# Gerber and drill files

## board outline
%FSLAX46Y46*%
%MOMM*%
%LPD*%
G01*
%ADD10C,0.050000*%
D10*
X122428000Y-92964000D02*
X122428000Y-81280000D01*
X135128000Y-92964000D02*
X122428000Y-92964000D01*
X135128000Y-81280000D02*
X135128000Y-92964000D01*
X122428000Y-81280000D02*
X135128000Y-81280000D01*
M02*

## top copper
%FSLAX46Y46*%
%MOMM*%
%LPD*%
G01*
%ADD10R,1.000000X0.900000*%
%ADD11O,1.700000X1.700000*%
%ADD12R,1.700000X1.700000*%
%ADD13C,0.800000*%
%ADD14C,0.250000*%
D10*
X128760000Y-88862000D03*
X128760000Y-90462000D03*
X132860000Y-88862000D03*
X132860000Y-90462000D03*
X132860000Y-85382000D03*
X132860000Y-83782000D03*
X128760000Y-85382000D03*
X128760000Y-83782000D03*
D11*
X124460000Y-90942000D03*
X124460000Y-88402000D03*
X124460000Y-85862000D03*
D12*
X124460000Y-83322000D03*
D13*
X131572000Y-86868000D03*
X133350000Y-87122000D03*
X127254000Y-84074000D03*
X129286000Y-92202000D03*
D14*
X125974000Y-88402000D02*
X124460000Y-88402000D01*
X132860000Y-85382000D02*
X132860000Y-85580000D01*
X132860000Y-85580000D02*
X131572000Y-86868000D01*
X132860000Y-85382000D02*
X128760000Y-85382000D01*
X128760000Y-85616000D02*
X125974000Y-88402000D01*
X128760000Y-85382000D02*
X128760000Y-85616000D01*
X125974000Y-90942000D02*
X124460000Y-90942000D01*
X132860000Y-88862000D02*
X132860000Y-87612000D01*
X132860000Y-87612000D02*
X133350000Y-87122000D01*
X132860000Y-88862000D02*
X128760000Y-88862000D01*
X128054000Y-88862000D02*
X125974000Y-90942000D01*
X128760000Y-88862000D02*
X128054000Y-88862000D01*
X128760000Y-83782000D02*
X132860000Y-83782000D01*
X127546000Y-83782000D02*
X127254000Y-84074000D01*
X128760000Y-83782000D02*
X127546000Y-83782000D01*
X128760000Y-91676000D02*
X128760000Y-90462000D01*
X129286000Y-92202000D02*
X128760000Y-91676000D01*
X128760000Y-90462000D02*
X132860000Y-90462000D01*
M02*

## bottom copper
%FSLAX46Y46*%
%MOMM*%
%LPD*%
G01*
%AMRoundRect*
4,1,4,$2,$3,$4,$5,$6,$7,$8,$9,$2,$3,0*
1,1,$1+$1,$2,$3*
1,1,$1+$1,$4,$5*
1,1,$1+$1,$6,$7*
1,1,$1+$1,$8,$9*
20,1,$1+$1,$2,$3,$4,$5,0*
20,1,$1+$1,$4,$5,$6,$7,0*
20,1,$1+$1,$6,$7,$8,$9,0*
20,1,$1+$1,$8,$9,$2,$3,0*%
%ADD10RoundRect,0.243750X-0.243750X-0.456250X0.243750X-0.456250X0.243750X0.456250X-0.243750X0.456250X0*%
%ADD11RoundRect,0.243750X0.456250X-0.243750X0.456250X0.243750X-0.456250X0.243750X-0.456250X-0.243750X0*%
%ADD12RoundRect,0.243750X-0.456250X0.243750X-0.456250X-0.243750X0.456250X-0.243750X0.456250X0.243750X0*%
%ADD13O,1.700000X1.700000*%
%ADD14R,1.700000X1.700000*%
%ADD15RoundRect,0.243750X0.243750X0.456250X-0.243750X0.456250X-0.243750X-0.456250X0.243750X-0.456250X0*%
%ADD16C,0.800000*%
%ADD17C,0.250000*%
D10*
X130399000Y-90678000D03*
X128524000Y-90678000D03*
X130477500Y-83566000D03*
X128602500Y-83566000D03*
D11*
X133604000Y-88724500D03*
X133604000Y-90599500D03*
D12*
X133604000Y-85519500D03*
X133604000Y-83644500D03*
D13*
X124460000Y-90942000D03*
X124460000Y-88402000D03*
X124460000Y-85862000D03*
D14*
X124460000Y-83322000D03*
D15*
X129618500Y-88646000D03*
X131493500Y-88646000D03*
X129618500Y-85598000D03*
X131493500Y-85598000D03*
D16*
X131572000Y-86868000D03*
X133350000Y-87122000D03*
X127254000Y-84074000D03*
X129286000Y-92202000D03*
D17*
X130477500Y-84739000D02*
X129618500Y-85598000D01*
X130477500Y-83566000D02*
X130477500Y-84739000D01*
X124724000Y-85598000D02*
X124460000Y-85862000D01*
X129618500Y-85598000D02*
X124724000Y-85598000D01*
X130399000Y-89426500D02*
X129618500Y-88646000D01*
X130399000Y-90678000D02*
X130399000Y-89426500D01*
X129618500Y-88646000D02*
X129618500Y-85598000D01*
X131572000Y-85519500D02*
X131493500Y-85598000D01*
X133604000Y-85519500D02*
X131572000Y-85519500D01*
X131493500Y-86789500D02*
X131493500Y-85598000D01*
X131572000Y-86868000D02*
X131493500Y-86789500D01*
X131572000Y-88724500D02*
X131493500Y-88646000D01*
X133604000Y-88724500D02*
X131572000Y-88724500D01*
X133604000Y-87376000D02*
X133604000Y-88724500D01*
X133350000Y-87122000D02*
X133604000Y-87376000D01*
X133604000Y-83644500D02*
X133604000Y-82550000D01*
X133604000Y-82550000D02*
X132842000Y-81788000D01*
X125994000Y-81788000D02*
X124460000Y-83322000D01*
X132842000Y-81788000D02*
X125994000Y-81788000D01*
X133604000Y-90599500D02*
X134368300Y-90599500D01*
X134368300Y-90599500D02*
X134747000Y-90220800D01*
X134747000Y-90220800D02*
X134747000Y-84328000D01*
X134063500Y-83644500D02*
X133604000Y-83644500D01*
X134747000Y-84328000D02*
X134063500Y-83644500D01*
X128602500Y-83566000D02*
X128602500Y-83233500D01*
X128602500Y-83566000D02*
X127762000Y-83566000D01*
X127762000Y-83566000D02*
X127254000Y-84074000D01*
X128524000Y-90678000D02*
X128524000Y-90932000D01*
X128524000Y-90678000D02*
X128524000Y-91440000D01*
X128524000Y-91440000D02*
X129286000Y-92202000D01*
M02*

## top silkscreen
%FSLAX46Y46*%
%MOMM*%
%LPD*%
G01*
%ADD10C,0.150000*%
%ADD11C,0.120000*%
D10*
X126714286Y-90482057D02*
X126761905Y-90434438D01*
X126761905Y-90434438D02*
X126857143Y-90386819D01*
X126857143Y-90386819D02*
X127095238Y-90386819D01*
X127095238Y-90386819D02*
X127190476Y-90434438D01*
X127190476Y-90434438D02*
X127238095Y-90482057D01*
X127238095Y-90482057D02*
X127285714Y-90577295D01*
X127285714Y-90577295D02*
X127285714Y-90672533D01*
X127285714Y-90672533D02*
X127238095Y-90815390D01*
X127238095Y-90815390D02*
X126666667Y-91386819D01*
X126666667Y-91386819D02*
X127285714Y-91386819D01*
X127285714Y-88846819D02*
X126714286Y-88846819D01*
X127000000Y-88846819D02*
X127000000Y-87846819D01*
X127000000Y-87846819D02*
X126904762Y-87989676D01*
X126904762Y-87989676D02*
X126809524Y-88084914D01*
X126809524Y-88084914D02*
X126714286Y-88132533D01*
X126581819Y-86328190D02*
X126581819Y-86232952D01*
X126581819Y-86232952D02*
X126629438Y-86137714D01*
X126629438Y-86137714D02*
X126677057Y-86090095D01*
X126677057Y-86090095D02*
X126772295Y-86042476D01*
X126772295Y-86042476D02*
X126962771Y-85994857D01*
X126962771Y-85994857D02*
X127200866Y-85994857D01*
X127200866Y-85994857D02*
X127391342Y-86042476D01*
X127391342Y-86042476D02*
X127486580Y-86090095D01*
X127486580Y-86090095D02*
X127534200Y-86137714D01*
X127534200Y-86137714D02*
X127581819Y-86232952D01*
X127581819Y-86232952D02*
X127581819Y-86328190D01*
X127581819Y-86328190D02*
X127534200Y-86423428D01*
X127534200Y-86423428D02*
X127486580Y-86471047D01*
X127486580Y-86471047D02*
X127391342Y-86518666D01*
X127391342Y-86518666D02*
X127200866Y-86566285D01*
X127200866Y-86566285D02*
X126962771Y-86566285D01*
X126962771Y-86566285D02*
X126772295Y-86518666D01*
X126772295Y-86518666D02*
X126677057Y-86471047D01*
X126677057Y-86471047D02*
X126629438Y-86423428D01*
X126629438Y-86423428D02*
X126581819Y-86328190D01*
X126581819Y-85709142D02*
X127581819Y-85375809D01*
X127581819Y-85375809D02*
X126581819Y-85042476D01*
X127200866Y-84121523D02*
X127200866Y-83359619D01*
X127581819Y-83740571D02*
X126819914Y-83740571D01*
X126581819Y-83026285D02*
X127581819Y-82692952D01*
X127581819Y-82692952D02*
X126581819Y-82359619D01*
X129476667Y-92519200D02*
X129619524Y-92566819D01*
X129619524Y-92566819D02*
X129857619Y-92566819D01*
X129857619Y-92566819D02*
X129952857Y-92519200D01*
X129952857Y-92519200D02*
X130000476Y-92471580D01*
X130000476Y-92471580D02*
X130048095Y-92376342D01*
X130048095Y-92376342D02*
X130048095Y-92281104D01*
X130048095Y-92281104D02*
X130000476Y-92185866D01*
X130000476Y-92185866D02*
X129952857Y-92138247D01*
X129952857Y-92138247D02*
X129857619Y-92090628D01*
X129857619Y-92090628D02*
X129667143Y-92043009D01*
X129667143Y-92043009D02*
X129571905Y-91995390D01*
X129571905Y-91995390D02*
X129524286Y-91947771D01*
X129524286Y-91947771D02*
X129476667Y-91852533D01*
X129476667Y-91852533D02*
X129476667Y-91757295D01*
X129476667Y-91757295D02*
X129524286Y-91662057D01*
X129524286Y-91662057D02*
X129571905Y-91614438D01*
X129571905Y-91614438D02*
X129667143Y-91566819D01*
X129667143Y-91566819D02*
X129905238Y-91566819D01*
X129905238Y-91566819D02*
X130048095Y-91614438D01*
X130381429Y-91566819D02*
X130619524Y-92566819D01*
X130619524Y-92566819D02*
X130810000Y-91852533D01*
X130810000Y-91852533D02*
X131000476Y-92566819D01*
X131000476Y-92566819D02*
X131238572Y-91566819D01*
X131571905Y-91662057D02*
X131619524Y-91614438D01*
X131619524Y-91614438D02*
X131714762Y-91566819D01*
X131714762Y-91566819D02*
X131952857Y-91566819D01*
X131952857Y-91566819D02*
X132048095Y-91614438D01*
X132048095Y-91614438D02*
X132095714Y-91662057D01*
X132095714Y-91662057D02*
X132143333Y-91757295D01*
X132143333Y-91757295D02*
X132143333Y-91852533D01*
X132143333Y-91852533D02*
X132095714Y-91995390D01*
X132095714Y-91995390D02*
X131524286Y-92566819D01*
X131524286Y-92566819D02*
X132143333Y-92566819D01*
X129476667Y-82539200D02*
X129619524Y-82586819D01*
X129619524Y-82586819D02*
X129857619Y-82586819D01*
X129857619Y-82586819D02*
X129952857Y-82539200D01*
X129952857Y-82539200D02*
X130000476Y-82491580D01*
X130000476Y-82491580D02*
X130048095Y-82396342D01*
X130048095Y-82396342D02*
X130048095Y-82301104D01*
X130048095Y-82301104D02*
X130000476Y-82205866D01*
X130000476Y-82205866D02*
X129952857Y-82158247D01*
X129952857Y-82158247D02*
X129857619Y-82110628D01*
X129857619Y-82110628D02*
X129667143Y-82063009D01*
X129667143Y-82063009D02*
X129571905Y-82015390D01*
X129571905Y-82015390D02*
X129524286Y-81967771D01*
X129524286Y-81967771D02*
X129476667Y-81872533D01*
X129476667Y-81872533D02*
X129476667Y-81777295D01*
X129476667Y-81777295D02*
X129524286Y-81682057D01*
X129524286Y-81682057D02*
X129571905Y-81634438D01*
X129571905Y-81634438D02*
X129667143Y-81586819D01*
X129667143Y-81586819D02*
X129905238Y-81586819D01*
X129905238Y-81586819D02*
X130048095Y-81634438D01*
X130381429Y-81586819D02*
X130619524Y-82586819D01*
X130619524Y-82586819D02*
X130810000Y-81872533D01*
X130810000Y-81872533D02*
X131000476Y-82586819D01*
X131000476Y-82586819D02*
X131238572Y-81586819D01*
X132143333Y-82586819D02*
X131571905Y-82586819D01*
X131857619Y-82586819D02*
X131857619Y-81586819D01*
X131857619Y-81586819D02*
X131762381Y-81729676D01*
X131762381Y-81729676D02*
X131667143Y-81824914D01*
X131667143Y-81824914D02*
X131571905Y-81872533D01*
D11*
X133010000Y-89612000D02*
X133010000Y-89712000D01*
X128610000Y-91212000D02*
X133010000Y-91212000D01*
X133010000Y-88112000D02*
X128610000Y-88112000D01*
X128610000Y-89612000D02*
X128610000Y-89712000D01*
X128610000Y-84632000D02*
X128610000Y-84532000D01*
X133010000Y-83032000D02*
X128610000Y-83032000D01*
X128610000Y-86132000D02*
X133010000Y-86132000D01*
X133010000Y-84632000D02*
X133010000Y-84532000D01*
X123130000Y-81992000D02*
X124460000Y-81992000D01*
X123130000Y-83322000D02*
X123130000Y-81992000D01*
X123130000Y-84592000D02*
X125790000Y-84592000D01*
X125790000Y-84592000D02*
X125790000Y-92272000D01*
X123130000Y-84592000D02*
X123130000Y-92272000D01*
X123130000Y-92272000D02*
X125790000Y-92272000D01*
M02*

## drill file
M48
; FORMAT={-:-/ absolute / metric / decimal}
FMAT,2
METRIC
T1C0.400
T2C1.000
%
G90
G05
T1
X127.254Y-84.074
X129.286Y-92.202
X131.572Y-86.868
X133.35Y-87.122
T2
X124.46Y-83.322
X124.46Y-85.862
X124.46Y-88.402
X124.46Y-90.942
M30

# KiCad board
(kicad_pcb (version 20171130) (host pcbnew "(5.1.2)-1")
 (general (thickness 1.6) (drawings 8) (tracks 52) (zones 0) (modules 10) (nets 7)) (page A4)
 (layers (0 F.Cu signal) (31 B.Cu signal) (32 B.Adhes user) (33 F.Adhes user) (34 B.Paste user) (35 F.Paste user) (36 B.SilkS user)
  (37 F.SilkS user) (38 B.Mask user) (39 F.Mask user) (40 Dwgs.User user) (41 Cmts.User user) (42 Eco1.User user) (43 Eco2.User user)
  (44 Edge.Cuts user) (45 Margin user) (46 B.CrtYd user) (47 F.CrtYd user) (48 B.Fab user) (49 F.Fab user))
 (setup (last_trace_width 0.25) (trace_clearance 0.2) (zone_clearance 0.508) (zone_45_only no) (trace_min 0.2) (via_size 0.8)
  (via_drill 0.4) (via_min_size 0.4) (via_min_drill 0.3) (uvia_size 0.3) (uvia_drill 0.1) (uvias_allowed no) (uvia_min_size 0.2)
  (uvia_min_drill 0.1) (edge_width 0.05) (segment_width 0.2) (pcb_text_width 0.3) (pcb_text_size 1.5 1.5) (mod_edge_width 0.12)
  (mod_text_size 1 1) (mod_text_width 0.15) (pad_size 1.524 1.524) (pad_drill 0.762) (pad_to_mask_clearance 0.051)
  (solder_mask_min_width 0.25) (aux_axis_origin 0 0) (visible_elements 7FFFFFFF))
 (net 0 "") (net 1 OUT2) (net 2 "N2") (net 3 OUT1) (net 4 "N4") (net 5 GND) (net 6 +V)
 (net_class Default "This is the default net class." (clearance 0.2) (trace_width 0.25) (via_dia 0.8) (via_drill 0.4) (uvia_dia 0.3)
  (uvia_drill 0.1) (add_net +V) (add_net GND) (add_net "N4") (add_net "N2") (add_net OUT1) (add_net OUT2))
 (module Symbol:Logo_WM (layer B.Cu) (at 127.381 87.122 270)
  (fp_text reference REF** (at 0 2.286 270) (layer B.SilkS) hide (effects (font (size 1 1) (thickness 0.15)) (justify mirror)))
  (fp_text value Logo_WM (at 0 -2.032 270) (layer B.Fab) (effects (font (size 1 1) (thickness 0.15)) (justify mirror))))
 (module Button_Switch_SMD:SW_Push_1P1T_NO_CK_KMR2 (layer F.Cu) (at 130.81 89.662 180)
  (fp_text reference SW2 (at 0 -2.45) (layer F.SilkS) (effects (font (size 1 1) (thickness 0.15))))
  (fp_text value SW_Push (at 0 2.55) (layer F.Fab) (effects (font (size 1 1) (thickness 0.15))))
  (fp_line (start -2.2 0.05) (end -2.2 -0.05) (layer F.SilkS) (width 0.12))
  (fp_line (start 2.2 -1.55) (end -2.2 -1.55) (layer F.SilkS) (width 0.12))
  (fp_line (start -2.2 1.55) (end 2.2 1.55) (layer F.SilkS) (width 0.12))
  (fp_line (start 2.2 0.05) (end 2.2 -0.05) (layer F.SilkS) (width 0.12))
  (pad 2 smd rect (at 2.05 0.8 270) (size 0.9 1) (layers F.Cu F.Paste F.Mask) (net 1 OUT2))
  (pad 1 smd rect (at 2.05 -0.8 270) (size 0.9 1) (layers F.Cu F.Paste F.Mask) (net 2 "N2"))
  (pad 2 smd rect (at -2.05 0.8 270) (size 0.9 1) (layers F.Cu F.Paste F.Mask) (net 1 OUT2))
  (pad 1 smd rect (at -2.05 -0.8 270) (size 0.9 1) (layers F.Cu F.Paste F.Mask) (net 2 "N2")))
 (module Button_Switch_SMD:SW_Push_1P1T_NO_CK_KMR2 (layer F.Cu) (at 130.81 84.582)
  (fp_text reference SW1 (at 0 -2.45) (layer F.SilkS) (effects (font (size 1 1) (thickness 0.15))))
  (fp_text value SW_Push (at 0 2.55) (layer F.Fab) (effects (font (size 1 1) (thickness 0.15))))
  (fp_line (start -2.2 0.05) (end -2.2 -0.05) (layer F.SilkS) (width 0.12))
  (fp_line (start 2.2 -1.55) (end -2.2 -1.55) (layer F.SilkS) (width 0.12))
  (fp_line (start -2.2 1.55) (end 2.2 1.55) (layer F.SilkS) (width 0.12))
  (fp_line (start 2.2 0.05) (end 2.2 -0.05) (layer F.SilkS) (width 0.12))
  (pad 2 smd rect (at 2.05 0.8 90) (size 0.9 1) (layers F.Cu F.Paste F.Mask) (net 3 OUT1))
  (pad 1 smd rect (at 2.05 -0.8 90) (size 0.9 1) (layers F.Cu F.Paste F.Mask) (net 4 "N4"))
  (pad 2 smd rect (at -2.05 0.8 90) (size 0.9 1) (layers F.Cu F.Paste F.Mask) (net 3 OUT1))
  (pad 1 smd rect (at -2.05 -0.8 90) (size 0.9 1) (layers F.Cu F.Paste F.Mask) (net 4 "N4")))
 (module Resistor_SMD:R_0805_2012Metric (layer B.Cu) (at 129.4615 90.678)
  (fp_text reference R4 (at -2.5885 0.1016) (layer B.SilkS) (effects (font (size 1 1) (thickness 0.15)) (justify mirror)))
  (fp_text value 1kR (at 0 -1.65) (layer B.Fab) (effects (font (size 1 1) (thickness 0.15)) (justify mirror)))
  (pad 2 smd roundrect (at 0.9375 0) (size 0.975 1.4) (layers B.Cu B.Paste B.Mask) (roundrect_rratio 0.25) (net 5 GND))
  (pad 1 smd roundrect (at -0.9375 0) (size 0.975 1.4) (layers B.Cu B.Paste B.Mask) (roundrect_rratio 0.25) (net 2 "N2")))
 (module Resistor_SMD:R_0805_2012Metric (layer B.Cu) (at 129.54 83.566)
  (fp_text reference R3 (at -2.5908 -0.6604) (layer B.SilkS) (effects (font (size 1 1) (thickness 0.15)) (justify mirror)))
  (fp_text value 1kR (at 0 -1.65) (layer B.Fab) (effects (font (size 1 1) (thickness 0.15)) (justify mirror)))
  (pad 2 smd roundrect (at 0.9375 0) (size 0.975 1.4) (layers B.Cu B.Paste B.Mask) (roundrect_rratio 0.25) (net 5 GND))
  (pad 1 smd roundrect (at -0.9375 0) (size 0.975 1.4) (layers B.Cu B.Paste B.Mask) (roundrect_rratio 0.25) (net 4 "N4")))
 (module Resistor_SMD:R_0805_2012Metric (layer B.Cu) (at 133.604 89.662 90)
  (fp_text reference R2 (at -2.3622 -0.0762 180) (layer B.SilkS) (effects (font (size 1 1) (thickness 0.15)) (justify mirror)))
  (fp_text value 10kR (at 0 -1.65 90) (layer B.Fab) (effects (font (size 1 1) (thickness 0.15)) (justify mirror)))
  (pad 2 smd roundrect (at 0.9375 0 90) (size 0.975 1.4) (layers B.Cu B.Paste B.Mask) (roundrect_rratio 0.25) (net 1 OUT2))
  (pad 1 smd roundrect (at -0.9375 0 90) (size 0.975 1.4) (layers B.Cu B.Paste B.Mask) (roundrect_rratio 0.25) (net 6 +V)))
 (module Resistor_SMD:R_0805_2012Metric (layer B.Cu) (at 133.604 84.582 270)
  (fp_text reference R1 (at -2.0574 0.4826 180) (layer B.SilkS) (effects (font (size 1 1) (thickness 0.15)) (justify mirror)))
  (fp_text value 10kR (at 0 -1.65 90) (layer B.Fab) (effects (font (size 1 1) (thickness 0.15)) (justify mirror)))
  (pad 2 smd roundrect (at 0.9375 0 270) (size 0.975 1.4) (layers B.Cu B.Paste B.Mask) (roundrect_rratio 0.25) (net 3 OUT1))
  (pad 1 smd roundrect (at -0.9375 0 270) (size 0.975 1.4) (layers B.Cu B.Paste B.Mask) (roundrect_rratio 0.25) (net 6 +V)))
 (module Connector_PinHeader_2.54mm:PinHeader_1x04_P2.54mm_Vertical (layer F.Cu) (at 124.46 83.322)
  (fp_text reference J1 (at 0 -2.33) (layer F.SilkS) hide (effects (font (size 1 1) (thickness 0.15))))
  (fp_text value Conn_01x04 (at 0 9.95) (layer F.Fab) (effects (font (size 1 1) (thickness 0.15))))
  (fp_line (start -1.33 -1.33) (end 0 -1.33) (layer F.SilkS) (width 0.12))
  (fp_line (start -1.33 0) (end -1.33 -1.33) (layer F.SilkS) (width 0.12))
  (fp_line (start -1.33 1.27) (end 1.33 1.27) (layer F.SilkS) (width 0.12))
  (fp_line (start 1.33 1.27) (end 1.33 8.95) (layer F.SilkS) (width 0.12))
  (fp_line (start -1.33 1.27) (end -1.33 8.95) (layer F.SilkS) (width 0.12))
  (fp_line (start -1.33 8.95) (end 1.33 8.95) (layer F.SilkS) (width 0.12))
  (pad 4 thru_hole oval (at 0 7.62) (size 1.7 1.7) (drill 1) (layers *.Cu *.Mask) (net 1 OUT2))
  (pad 3 thru_hole oval (at 0 5.08) (size 1.7 1.7) (drill 1) (layers *.Cu *.Mask) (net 3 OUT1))
  (pad 2 thru_hole oval (at 0 2.54) (size 1.7 1.7) (drill 1) (layers *.Cu *.Mask) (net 5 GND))
  (pad 1 thru_hole rect (at 0 0) (size 1.7 1.7) (drill 1) (layers *.Cu *.Mask) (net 6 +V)))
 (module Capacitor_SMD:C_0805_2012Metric (layer B.Cu) (at 130.556 88.646 180)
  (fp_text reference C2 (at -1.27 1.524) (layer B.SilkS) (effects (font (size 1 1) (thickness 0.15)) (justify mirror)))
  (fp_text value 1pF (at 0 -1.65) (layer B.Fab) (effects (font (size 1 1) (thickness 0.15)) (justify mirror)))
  (pad 2 smd roundrect (at 0.9375 0 180) (size 0.975 1.4) (layers B.Cu B.Paste B.Mask) (roundrect_rratio 0.25) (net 5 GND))
  (pad 1 smd roundrect (at -0.9375 0 180) (size 0.975 1.4) (layers B.Cu B.Paste B.Mask) (roundrect_rratio 0.25) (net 1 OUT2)))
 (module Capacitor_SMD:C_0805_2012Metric (layer B.Cu) (at 130.556 85.598 180)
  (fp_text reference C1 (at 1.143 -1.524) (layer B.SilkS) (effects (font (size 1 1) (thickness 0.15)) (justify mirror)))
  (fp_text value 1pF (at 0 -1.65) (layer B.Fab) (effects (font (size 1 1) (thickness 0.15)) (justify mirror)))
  (pad 2 smd roundrect (at 0.9375 0 180) (size 0.975 1.4) (layers B.Cu B.Paste B.Mask) (roundrect_rratio 0.25) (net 5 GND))
  (pad 1 smd roundrect (at -0.9375 0 180) (size 0.975 1.4) (layers B.Cu B.Paste B.Mask) (roundrect_rratio 0.25) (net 3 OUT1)))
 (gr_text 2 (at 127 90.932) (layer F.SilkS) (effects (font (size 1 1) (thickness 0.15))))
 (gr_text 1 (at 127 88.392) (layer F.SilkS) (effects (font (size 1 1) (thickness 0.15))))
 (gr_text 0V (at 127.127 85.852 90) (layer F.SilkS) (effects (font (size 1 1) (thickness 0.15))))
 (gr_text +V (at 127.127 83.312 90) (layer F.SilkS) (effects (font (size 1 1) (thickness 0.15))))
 (gr_line (start 122.428 92.964) (end 122.428 81.28) (layer Edge.Cuts) (width 0.05))
 (gr_line (start 135.128 92.964) (end 122.428 92.964) (layer Edge.Cuts) (width 0.05))
 (gr_line (start 135.128 81.28) (end 135.128 92.964) (layer Edge.Cuts) (width 0.05))
 (gr_line (start 122.428 81.28) (end 135.128 81.28) (layer Edge.Cuts) (width 0.05))
 (segment (start 130.4775 84.739) (end 129.6185 85.598) (width 0.25) (layer B.Cu) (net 5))
 (segment (start 130.4775 83.566) (end 130.4775 84.739) (width 0.25) (layer B.Cu) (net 5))
 (segment (start 124.724 85.598) (end 124.46 85.862) (width 0.25) (layer B.Cu) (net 5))
 (segment (start 129.6185 85.598) (end 124.724 85.598) (width 0.25) (layer B.Cu) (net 5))
 (segment (start 130.399 89.4265) (end 129.6185 88.646) (width 0.25) (layer B.Cu) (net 5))
 (segment (start 130.399 90.678) (end 130.399 89.4265) (width 0.25) (layer B.Cu) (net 5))
 (segment (start 129.6185 88.646) (end 129.6185 85.598) (width 0.25) (layer B.Cu) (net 5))
 (segment (start 131.572 85.5195) (end 131.4935 85.598) (width 0.25) (layer B.Cu) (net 3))
 (segment (start 133.604 85.5195) (end 131.572 85.5195) (width 0.25) (layer B.Cu) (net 3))
 (segment (start 125.974 88.402) (end 124.46 88.402) (width 0.25) (layer F.Cu) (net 3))
 (via (at 131.572 86.868) (size 0.8) (drill 0.4) (layers F.Cu B.Cu) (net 3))
 (segment (start 132.86 85.382) (end 132.86 85.58) (width 0.25) (layer F.Cu) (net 3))
 (segment (start 132.86 85.58) (end 131.572 86.868) (width 0.25) (layer F.Cu) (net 3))
 (segment (start 131.4935 86.7895) (end 131.4935 85.598) (width 0.25) (layer B.Cu) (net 3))
 (segment (start 131.572 86.868) (end 131.4935 86.7895) (width 0.25) (layer B.Cu) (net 3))
 (segment (start 132.86 85.382) (end 128.76 85.382) (width 0.25) (layer F.Cu) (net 3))
 (segment (start 128.76 85.616) (end 125.974 88.402) (width 0.25) (layer F.Cu) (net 3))
 (segment (start 128.76 85.382) (end 128.76 85.616) (width 0.25) (layer F.Cu) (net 3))
 (segment (start 131.572 88.7245) (end 131.4935 88.646) (width 0.25) (layer B.Cu) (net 1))
 (segment (start 133.604 88.7245) (end 131.572 88.7245) (width 0.25) (layer B.Cu) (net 1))
 (segment (start 125.974 90.942) (end 124.46 90.942) (width 0.25) (layer F.Cu) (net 1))
 (via (at 133.35 87.122) (size 0.8) (drill 0.4) (layers F.Cu B.Cu) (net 1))
 (segment (start 132.86 88.862) (end 132.86 87.612) (width 0.25) (layer F.Cu) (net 1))
 (segment (start 132.86 87.612) (end 133.35 87.122) (width 0.25) (layer F.Cu) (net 1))
 (segment (start 133.604 87.376) (end 133.604 88.7245) (width 0.25) (layer B.Cu) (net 1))
 (segment (start 133.35 87.122) (end 133.604 87.376) (width 0.25) (layer B.Cu) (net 1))
 (segment (start 132.86 88.862) (end 128.76 88.862) (width 0.25) (layer F.Cu) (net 1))
 (segment (start 128.054 88.862) (end 125.974 90.942) (width 0.25) (layer F.Cu) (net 1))
 (segment (start 128.76 88.862) (end 128.054 88.862) (width 0.25) (layer F.Cu) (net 1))
 (segment (start 133.604 83.6445) (end 133.604 82.55) (width 0.25) (layer B.Cu) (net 6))
 (segment (start 133.604 82.55) (end 132.842 81.788) (width 0.25) (layer B.Cu) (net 6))
 (segment (start 125.994 81.788) (end 124.46 83.322) (width 0.25) (layer B.Cu) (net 6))
 (segment (start 132.842 81.788) (end 125.994 81.788) (width 0.25) (layer B.Cu) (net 6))
 (segment (start 133.604 90.5995) (end 134.3683 90.5995) (width 0.25) (layer B.Cu) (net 6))
 (segment (start 134.3683 90.5995) (end 134.747 90.2208) (width 0.25) (layer B.Cu) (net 6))
 (segment (start 134.747 90.2208) (end 134.747 84.328) (width 0.25) (layer B.Cu) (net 6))
 (segment (start 134.0635 83.6445) (end 133.604 83.6445) (width 0.25) (layer B.Cu) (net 6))
 (segment (start 134.747 84.328) (end 134.0635 83.6445) (width 0.25) (layer B.Cu) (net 6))
 (segment (start 128.6025 83.566) (end 128.6025 83.2335) (width 0.25) (layer B.Cu) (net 4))
 (via (at 127.254 84.074) (size 0.8) (drill 0.4) (layers F.Cu B.Cu) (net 4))
 (segment (start 128.6025 83.566) (end 127.762 83.566) (width 0.25) (layer B.Cu) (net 4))
 (segment (start 127.762 83.566) (end 127.254 84.074) (width 0.25) (layer B.Cu) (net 4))
 (segment (start 128.76 83.782) (end 132.86 83.782) (width 0.25) (layer F.Cu) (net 4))
 (segment (start 127.546 83.782) (end 127.254 84.074) (width 0.25) (layer F.Cu) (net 4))
 (segment (start 128.76 83.782) (end 127.546 83.782) (width 0.25) (layer F.Cu) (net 4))
 (segment (start 128.524 90.678) (end 128.524 90.932) (width 0.25) (layer B.Cu) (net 2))
 (via (at 129.286 92.202) (size 0.8) (drill 0.4) (layers F.Cu B.Cu) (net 2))
 (segment (start 128.524 90.678) (end 128.524 91.44) (width 0.25) (layer B.Cu) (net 2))
 (segment (start 128.524 91.44) (end 129.286 92.202) (width 0.25) (layer B.Cu) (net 2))
 (segment (start 128.76 91.676) (end 128.76 90.462) (width 0.25) (layer F.Cu) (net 2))
 (segment (start 129.286 92.202) (end 128.76 91.676) (width 0.25) (layer F.Cu) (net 2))
 (segment (start 128.76 90.462) (end 132.86 90.462) (width 0.25) (layer F.Cu) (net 2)))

